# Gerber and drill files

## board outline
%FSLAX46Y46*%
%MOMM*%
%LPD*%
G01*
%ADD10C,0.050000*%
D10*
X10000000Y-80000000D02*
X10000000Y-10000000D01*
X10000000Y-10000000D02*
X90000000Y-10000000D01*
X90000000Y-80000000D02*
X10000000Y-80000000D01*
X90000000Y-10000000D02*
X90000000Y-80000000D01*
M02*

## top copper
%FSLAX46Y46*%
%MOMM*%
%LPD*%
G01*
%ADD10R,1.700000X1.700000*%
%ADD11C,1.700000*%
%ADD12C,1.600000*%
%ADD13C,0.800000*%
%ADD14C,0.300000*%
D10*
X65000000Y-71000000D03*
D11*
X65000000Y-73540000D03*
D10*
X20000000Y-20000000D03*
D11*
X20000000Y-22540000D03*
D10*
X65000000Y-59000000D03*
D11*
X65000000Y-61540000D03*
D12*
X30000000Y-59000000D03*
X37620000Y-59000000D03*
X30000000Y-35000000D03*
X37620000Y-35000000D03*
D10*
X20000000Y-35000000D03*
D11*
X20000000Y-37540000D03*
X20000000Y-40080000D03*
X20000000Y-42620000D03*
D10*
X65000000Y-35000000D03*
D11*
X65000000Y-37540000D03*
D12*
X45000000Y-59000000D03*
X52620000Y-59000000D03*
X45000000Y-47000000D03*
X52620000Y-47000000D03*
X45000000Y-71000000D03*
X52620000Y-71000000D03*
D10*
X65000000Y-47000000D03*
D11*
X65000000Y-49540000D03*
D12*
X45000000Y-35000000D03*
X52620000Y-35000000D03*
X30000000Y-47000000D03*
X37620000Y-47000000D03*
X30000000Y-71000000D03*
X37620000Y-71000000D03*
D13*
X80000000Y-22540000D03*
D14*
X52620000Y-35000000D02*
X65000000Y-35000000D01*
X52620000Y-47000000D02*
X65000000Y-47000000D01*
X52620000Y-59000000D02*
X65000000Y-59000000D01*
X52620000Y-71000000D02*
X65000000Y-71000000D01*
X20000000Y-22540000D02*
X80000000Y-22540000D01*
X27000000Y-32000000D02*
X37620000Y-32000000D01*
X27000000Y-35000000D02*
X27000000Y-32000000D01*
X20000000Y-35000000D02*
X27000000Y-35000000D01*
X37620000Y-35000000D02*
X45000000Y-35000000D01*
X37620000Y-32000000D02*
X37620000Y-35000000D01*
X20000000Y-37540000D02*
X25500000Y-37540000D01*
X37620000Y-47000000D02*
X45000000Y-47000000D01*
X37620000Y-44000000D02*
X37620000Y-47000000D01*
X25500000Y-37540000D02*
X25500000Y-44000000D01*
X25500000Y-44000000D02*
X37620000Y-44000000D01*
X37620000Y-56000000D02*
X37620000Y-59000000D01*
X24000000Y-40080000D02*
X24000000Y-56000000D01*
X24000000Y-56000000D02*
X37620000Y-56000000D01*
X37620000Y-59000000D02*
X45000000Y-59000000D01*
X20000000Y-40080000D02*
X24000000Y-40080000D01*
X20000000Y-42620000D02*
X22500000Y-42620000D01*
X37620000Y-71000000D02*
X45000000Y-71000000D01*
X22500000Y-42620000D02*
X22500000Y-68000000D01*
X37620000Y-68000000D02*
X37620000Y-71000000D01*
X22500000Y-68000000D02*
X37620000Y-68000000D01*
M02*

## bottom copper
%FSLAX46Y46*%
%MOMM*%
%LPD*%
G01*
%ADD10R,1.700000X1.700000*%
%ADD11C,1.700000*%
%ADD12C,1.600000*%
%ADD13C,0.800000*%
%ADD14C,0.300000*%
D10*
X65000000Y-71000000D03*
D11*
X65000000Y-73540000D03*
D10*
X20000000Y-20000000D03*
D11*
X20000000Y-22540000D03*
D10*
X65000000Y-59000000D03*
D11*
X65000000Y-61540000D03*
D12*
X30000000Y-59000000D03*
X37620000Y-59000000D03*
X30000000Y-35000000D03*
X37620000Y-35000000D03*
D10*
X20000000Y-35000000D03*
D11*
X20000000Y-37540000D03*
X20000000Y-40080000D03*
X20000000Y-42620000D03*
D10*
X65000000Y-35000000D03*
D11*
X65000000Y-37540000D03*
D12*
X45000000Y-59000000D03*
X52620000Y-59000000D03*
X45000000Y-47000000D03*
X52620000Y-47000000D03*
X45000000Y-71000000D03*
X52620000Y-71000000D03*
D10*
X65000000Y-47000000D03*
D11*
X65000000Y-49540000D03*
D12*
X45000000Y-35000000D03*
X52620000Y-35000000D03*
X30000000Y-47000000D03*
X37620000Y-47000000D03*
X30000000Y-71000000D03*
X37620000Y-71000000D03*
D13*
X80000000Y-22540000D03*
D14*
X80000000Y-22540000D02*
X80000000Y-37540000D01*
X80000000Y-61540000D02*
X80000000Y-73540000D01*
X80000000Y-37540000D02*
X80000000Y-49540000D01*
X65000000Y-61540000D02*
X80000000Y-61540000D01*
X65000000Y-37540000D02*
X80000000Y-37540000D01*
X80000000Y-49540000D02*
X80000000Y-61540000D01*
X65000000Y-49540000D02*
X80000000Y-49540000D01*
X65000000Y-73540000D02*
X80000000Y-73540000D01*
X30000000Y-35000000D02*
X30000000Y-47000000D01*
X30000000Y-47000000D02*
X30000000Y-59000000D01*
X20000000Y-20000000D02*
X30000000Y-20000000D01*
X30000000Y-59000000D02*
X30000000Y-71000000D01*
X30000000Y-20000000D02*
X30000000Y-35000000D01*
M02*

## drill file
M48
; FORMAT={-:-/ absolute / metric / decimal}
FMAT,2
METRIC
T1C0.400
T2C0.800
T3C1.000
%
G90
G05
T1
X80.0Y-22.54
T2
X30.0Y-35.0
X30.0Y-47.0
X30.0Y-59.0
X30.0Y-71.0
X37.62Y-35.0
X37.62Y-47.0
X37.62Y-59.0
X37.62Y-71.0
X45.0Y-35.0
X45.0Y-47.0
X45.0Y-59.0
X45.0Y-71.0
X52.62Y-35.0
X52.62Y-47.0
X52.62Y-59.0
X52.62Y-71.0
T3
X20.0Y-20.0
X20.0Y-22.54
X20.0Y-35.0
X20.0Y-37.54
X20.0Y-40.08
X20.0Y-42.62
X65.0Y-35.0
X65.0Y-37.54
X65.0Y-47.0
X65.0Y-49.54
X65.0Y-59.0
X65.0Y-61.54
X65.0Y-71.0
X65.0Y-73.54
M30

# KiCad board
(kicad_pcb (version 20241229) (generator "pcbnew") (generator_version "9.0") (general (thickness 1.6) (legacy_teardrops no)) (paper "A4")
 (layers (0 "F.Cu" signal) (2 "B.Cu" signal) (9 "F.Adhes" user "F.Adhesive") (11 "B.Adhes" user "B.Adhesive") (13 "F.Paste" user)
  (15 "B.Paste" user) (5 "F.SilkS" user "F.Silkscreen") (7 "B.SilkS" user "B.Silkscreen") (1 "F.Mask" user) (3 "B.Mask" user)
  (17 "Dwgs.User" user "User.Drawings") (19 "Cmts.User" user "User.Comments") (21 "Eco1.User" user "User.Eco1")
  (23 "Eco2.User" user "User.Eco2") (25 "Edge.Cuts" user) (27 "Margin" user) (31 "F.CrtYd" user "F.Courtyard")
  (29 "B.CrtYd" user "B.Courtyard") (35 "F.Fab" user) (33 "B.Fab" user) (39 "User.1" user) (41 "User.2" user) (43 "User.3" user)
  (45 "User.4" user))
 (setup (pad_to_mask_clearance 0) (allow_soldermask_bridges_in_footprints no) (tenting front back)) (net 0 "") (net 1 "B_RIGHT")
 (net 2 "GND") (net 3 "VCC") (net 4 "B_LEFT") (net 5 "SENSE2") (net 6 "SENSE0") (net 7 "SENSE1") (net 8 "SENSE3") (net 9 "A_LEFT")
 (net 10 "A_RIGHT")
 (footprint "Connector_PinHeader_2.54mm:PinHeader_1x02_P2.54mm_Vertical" (layer "F.Cu") (at 65 71)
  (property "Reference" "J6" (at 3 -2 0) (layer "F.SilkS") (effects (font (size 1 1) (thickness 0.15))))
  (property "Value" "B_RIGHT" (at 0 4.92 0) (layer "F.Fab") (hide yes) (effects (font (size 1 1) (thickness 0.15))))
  (pad "1" thru_hole rect (at 0 0) (size 1.7 1.7) (drill 1) (layers "*.Cu" "*.Mask") (remove_unused_layers no) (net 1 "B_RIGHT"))
  (pad "2" thru_hole circle (at 0 2.54) (size 1.7 1.7) (drill 1) (layers "*.Cu" "*.Mask") (remove_unused_layers no) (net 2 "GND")))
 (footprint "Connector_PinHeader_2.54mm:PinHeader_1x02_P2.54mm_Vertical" (layer "F.Cu") (at 20 20)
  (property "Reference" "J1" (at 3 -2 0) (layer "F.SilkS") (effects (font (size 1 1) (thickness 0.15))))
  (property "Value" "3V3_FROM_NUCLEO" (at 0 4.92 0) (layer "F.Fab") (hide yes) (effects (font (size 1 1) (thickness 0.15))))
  (pad "1" thru_hole rect (at 0 0) (size 1.7 1.7) (drill 1) (layers "*.Cu" "*.Mask") (remove_unused_layers no) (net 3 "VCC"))
  (pad "2" thru_hole circle (at 0 2.54) (size 1.7 1.7) (drill 1) (layers "*.Cu" "*.Mask") (remove_unused_layers no) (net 2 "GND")))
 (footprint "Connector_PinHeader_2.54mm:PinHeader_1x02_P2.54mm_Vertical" (layer "F.Cu") (at 65 59)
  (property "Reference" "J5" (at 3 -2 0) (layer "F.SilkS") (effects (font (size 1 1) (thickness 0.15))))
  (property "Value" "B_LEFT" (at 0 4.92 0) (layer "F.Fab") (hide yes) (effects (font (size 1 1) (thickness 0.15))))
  (pad "1" thru_hole rect (at 0 0) (size 1.7 1.7) (drill 1) (layers "*.Cu" "*.Mask") (remove_unused_layers no) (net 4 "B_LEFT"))
  (pad "2" thru_hole circle (at 0 2.54) (size 1.7 1.7) (drill 1) (layers "*.Cu" "*.Mask") (remove_unused_layers no) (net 2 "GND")))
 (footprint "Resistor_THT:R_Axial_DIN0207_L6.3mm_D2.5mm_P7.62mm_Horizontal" (layer "F.Cu") (at 30 59)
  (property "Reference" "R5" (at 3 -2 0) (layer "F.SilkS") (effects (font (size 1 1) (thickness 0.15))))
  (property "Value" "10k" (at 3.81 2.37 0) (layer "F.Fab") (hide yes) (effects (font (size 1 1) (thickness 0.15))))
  (pad "1" thru_hole circle (at 0 0) (size 1.6 1.6) (drill 0.8) (layers "*.Cu" "*.Mask") (remove_unused_layers no) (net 3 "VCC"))
  (pad "2" thru_hole circle (at 7.62 0) (size 1.6 1.6) (drill 0.8) (layers "*.Cu" "*.Mask") (remove_unused_layers no) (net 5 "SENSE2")))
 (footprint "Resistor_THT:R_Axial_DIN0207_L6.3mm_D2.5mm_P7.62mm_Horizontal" (layer "F.Cu") (at 30 35)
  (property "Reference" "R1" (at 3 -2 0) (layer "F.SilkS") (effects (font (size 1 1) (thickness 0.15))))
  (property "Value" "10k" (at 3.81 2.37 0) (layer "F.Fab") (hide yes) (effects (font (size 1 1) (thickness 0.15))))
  (pad "1" thru_hole circle (at 0 0) (size 1.6 1.6) (drill 0.8) (layers "*.Cu" "*.Mask") (remove_unused_layers no) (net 3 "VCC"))
  (pad "2" thru_hole circle (at 7.62 0) (size 1.6 1.6) (drill 0.8) (layers "*.Cu" "*.Mask") (remove_unused_layers no) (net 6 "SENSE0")))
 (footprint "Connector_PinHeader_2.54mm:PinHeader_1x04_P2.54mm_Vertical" (layer "F.Cu") (at 20 35)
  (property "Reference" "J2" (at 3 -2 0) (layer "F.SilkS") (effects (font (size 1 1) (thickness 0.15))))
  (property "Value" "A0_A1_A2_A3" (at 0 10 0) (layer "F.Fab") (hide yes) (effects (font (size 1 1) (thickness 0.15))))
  (pad "1" thru_hole rect (at 0 0) (size 1.7 1.7) (drill 1) (layers "*.Cu" "*.Mask") (remove_unused_layers no) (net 6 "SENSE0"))
  (pad "2" thru_hole circle (at 0 2.54) (size 1.7 1.7) (drill 1) (layers "*.Cu" "*.Mask") (remove_unused_layers no) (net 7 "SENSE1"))
  (pad "3" thru_hole circle (at 0 5.08) (size 1.7 1.7) (drill 1) (layers "*.Cu" "*.Mask") (remove_unused_layers no) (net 5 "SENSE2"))
  (pad "4" thru_hole circle (at 0 7.62) (size 1.7 1.7) (drill 1) (layers "*.Cu" "*.Mask") (remove_unused_layers no) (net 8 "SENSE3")))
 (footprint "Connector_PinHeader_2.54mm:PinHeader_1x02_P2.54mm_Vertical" (layer "F.Cu") (at 65 35)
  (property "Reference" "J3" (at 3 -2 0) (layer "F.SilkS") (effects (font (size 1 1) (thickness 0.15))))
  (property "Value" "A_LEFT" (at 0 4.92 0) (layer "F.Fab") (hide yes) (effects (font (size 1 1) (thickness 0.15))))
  (pad "1" thru_hole rect (at 0 0) (size 1.7 1.7) (drill 1) (layers "*.Cu" "*.Mask") (remove_unused_layers no) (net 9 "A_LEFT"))
  (pad "2" thru_hole circle (at 0 2.54) (size 1.7 1.7) (drill 1) (layers "*.Cu" "*.Mask") (remove_unused_layers no) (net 2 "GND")))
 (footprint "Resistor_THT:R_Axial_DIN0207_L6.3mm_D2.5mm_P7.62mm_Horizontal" (layer "F.Cu") (at 45 59)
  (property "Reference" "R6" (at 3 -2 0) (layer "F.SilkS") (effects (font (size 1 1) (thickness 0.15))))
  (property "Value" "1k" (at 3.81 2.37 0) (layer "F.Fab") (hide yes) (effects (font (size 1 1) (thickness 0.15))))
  (pad "1" thru_hole circle (at 0 0) (size 1.6 1.6) (drill 0.8) (layers "*.Cu" "*.Mask") (remove_unused_layers no) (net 5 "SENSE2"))
  (pad "2" thru_hole circle (at 7.62 0) (size 1.6 1.6) (drill 0.8) (layers "*.Cu" "*.Mask") (remove_unused_layers no) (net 4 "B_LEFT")))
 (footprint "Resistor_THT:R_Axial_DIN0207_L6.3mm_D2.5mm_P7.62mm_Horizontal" (layer "F.Cu") (at 45 47)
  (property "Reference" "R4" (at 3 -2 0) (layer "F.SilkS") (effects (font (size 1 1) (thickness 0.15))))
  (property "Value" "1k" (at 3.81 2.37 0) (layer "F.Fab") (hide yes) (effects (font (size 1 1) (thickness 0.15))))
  (pad "1" thru_hole circle (at 0 0) (size 1.6 1.6) (drill 0.8) (layers "*.Cu" "*.Mask") (remove_unused_layers no) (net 7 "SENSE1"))
  (pad "2" thru_hole circle (at 7.62 0) (size 1.6 1.6) (drill 0.8) (layers "*.Cu" "*.Mask") (remove_unused_layers no) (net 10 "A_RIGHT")))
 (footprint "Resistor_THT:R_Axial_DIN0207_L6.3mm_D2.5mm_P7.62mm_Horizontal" (layer "F.Cu") (at 45 71)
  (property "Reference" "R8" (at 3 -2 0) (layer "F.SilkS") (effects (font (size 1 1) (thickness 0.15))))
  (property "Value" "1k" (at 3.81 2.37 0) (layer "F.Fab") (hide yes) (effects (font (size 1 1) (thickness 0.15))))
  (pad "1" thru_hole circle (at 0 0) (size 1.6 1.6) (drill 0.8) (layers "*.Cu" "*.Mask") (remove_unused_layers no) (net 8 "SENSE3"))
  (pad "2" thru_hole circle (at 7.62 0) (size 1.6 1.6) (drill 0.8) (layers "*.Cu" "*.Mask") (remove_unused_layers no) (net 1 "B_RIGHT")))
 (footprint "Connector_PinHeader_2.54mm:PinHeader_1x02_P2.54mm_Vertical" (layer "F.Cu") (at 65 47)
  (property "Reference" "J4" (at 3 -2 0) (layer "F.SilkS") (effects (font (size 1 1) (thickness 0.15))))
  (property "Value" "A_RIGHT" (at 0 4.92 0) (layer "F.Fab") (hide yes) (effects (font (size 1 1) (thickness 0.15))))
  (pad "1" thru_hole rect (at 0 0) (size 1.7 1.7) (drill 1) (layers "*.Cu" "*.Mask") (remove_unused_layers no) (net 10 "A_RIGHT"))
  (pad "2" thru_hole circle (at 0 2.54) (size 1.7 1.7) (drill 1) (layers "*.Cu" "*.Mask") (remove_unused_layers no) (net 2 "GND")))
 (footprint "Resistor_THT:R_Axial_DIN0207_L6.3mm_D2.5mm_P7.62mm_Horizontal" (layer "F.Cu") (at 45 35)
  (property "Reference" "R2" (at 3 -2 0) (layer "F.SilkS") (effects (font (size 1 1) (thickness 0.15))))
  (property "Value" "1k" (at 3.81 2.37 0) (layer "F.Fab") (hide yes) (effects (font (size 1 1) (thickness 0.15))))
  (pad "1" thru_hole circle (at 0 0) (size 1.6 1.6) (drill 0.8) (layers "*.Cu" "*.Mask") (remove_unused_layers no) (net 6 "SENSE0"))
  (pad "2" thru_hole circle (at 7.62 0) (size 1.6 1.6) (drill 0.8) (layers "*.Cu" "*.Mask") (remove_unused_layers no) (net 9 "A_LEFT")))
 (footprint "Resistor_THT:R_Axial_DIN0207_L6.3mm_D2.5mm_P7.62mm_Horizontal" (layer "F.Cu") (at 30 47)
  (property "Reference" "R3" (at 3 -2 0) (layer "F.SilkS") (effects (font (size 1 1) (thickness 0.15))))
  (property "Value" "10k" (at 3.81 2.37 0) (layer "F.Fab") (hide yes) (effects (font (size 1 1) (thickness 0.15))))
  (pad "1" thru_hole circle (at 0 0) (size 1.6 1.6) (drill 0.8) (layers "*.Cu" "*.Mask") (remove_unused_layers no) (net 3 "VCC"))
  (pad "2" thru_hole circle (at 7.62 0) (size 1.6 1.6) (drill 0.8) (layers "*.Cu" "*.Mask") (remove_unused_layers no) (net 7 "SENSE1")))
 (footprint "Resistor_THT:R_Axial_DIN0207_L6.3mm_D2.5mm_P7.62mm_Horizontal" (layer "F.Cu") (at 30 71)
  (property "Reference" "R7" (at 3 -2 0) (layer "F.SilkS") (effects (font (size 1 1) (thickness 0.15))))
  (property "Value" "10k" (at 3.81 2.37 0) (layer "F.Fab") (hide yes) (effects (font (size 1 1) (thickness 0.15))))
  (pad "1" thru_hole circle (at 0 0) (size 1.6 1.6) (drill 0.8) (layers "*.Cu" "*.Mask") (remove_unused_layers no) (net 3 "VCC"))
  (pad "2" thru_hole circle (at 7.62 0) (size 1.6 1.6) (drill 0.8) (layers "*.Cu" "*.Mask") (remove_unused_layers no) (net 8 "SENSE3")))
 (gr_line (start 10 80) (end 10 10) (stroke (width 0.05) (type default)) (layer "Edge.Cuts"))
 (gr_line (start 10 10) (end 90 10) (stroke (width 0.05) (type default)) (layer "Edge.Cuts"))
 (gr_line (start 90 80) (end 10 80) (stroke (width 0.05) (type default)) (layer "Edge.Cuts"))
 (gr_line (start 90 10) (end 90 80) (stroke (width 0.05) (type default)) (layer "Edge.Cuts"))
 (segment (start 52.62 35) (end 65 35) (width 0.3) (layer "F.Cu") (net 9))
 (segment (start 52.62 47) (end 65 47) (width 0.3) (layer "F.Cu") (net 10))
 (segment (start 52.62 59) (end 65 59) (width 0.3) (layer "F.Cu") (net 4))
 (segment (start 52.62 71) (end 65 71) (width 0.3) (layer "F.Cu") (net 1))
 (segment (start 20 22.54) (end 80 22.54) (width 0.3) (layer "F.Cu") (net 2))
 (via (at 80 22.54) (size 0.8) (drill 0.4) (layers "F.Cu" "B.Cu") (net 2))
 (segment (start 80 22.54) (end 80 37.54) (width 0.3) (layer "B.Cu") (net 2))
 (segment (start 80 61.54) (end 80 73.54) (width 0.3) (layer "B.Cu") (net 2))
 (segment (start 80 37.54) (end 80 49.54) (width 0.3) (layer "B.Cu") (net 2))
 (segment (start 65 61.54) (end 80 61.54) (width 0.3) (layer "B.Cu") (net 2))
 (segment (start 65 37.54) (end 80 37.54) (width 0.3) (layer "B.Cu") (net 2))
 (segment (start 80 49.54) (end 80 61.54) (width 0.3) (layer "B.Cu") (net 2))
 (segment (start 65 49.54) (end 80 49.54) (width 0.3) (layer "B.Cu") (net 2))
 (segment (start 65 73.54) (end 80 73.54) (width 0.3) (layer "B.Cu") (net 2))
 (segment (start 27 32) (end 37.62 32) (width 0.3) (layer "F.Cu") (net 6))
 (segment (start 27 35) (end 27 32) (width 0.3) (layer "F.Cu") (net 6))
 (segment (start 20 35) (end 27 35) (width 0.3) (layer "F.Cu") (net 6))
 (segment (start 37.62 35) (end 45 35) (width 0.3) (layer "F.Cu") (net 6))
 (segment (start 37.62 32) (end 37.62 35) (width 0.3) (layer "F.Cu") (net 6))
 (segment (start 20 37.54) (end 25.5 37.54) (width 0.3) (layer "F.Cu") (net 7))
 (segment (start 37.62 47) (end 45 47) (width 0.3) (layer "F.Cu") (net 7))
 (segment (start 37.62 44) (end 37.62 47) (width 0.3) (layer "F.Cu") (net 7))
 (segment (start 25.5 37.54) (end 25.5 44) (width 0.3) (layer "F.Cu") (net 7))
 (segment (start 25.5 44) (end 37.62 44) (width 0.3) (layer "F.Cu") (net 7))
 (segment (start 37.62 56) (end 37.62 59) (width 0.3) (layer "F.Cu") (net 5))
 (segment (start 24 40.08) (end 24 56) (width 0.3) (layer "F.Cu") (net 5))
 (segment (start 24 56) (end 37.62 56) (width 0.3) (layer "F.Cu") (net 5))
 (segment (start 37.62 59) (end 45 59) (width 0.3) (layer "F.Cu") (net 5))
 (segment (start 20 40.08) (end 24 40.08) (width 0.3) (layer "F.Cu") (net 5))
 (segment (start 20 42.62) (end 22.5 42.62) (width 0.3) (layer "F.Cu") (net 8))
 (segment (start 37.62 71) (end 45 71) (width 0.3) (layer "F.Cu") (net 8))
 (segment (start 22.5 42.62) (end 22.5 68) (width 0.3) (layer "F.Cu") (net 8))
 (segment (start 37.62 68) (end 37.62 71) (width 0.3) (layer "F.Cu") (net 8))
 (segment (start 22.5 68) (end 37.62 68) (width 0.3) (layer "F.Cu") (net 8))
 (segment (start 30 35) (end 30 47) (width 0.3) (layer "B.Cu") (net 3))
 (segment (start 30 47) (end 30 59) (width 0.3) (layer "B.Cu") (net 3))
 (segment (start 20 20) (end 30 20) (width 0.3) (layer "B.Cu") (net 3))
 (segment (start 30 59) (end 30 71) (width 0.3) (layer "B.Cu") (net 3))
 (segment (start 30 20) (end 30 35) (width 0.3) (layer "B.Cu") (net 3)))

